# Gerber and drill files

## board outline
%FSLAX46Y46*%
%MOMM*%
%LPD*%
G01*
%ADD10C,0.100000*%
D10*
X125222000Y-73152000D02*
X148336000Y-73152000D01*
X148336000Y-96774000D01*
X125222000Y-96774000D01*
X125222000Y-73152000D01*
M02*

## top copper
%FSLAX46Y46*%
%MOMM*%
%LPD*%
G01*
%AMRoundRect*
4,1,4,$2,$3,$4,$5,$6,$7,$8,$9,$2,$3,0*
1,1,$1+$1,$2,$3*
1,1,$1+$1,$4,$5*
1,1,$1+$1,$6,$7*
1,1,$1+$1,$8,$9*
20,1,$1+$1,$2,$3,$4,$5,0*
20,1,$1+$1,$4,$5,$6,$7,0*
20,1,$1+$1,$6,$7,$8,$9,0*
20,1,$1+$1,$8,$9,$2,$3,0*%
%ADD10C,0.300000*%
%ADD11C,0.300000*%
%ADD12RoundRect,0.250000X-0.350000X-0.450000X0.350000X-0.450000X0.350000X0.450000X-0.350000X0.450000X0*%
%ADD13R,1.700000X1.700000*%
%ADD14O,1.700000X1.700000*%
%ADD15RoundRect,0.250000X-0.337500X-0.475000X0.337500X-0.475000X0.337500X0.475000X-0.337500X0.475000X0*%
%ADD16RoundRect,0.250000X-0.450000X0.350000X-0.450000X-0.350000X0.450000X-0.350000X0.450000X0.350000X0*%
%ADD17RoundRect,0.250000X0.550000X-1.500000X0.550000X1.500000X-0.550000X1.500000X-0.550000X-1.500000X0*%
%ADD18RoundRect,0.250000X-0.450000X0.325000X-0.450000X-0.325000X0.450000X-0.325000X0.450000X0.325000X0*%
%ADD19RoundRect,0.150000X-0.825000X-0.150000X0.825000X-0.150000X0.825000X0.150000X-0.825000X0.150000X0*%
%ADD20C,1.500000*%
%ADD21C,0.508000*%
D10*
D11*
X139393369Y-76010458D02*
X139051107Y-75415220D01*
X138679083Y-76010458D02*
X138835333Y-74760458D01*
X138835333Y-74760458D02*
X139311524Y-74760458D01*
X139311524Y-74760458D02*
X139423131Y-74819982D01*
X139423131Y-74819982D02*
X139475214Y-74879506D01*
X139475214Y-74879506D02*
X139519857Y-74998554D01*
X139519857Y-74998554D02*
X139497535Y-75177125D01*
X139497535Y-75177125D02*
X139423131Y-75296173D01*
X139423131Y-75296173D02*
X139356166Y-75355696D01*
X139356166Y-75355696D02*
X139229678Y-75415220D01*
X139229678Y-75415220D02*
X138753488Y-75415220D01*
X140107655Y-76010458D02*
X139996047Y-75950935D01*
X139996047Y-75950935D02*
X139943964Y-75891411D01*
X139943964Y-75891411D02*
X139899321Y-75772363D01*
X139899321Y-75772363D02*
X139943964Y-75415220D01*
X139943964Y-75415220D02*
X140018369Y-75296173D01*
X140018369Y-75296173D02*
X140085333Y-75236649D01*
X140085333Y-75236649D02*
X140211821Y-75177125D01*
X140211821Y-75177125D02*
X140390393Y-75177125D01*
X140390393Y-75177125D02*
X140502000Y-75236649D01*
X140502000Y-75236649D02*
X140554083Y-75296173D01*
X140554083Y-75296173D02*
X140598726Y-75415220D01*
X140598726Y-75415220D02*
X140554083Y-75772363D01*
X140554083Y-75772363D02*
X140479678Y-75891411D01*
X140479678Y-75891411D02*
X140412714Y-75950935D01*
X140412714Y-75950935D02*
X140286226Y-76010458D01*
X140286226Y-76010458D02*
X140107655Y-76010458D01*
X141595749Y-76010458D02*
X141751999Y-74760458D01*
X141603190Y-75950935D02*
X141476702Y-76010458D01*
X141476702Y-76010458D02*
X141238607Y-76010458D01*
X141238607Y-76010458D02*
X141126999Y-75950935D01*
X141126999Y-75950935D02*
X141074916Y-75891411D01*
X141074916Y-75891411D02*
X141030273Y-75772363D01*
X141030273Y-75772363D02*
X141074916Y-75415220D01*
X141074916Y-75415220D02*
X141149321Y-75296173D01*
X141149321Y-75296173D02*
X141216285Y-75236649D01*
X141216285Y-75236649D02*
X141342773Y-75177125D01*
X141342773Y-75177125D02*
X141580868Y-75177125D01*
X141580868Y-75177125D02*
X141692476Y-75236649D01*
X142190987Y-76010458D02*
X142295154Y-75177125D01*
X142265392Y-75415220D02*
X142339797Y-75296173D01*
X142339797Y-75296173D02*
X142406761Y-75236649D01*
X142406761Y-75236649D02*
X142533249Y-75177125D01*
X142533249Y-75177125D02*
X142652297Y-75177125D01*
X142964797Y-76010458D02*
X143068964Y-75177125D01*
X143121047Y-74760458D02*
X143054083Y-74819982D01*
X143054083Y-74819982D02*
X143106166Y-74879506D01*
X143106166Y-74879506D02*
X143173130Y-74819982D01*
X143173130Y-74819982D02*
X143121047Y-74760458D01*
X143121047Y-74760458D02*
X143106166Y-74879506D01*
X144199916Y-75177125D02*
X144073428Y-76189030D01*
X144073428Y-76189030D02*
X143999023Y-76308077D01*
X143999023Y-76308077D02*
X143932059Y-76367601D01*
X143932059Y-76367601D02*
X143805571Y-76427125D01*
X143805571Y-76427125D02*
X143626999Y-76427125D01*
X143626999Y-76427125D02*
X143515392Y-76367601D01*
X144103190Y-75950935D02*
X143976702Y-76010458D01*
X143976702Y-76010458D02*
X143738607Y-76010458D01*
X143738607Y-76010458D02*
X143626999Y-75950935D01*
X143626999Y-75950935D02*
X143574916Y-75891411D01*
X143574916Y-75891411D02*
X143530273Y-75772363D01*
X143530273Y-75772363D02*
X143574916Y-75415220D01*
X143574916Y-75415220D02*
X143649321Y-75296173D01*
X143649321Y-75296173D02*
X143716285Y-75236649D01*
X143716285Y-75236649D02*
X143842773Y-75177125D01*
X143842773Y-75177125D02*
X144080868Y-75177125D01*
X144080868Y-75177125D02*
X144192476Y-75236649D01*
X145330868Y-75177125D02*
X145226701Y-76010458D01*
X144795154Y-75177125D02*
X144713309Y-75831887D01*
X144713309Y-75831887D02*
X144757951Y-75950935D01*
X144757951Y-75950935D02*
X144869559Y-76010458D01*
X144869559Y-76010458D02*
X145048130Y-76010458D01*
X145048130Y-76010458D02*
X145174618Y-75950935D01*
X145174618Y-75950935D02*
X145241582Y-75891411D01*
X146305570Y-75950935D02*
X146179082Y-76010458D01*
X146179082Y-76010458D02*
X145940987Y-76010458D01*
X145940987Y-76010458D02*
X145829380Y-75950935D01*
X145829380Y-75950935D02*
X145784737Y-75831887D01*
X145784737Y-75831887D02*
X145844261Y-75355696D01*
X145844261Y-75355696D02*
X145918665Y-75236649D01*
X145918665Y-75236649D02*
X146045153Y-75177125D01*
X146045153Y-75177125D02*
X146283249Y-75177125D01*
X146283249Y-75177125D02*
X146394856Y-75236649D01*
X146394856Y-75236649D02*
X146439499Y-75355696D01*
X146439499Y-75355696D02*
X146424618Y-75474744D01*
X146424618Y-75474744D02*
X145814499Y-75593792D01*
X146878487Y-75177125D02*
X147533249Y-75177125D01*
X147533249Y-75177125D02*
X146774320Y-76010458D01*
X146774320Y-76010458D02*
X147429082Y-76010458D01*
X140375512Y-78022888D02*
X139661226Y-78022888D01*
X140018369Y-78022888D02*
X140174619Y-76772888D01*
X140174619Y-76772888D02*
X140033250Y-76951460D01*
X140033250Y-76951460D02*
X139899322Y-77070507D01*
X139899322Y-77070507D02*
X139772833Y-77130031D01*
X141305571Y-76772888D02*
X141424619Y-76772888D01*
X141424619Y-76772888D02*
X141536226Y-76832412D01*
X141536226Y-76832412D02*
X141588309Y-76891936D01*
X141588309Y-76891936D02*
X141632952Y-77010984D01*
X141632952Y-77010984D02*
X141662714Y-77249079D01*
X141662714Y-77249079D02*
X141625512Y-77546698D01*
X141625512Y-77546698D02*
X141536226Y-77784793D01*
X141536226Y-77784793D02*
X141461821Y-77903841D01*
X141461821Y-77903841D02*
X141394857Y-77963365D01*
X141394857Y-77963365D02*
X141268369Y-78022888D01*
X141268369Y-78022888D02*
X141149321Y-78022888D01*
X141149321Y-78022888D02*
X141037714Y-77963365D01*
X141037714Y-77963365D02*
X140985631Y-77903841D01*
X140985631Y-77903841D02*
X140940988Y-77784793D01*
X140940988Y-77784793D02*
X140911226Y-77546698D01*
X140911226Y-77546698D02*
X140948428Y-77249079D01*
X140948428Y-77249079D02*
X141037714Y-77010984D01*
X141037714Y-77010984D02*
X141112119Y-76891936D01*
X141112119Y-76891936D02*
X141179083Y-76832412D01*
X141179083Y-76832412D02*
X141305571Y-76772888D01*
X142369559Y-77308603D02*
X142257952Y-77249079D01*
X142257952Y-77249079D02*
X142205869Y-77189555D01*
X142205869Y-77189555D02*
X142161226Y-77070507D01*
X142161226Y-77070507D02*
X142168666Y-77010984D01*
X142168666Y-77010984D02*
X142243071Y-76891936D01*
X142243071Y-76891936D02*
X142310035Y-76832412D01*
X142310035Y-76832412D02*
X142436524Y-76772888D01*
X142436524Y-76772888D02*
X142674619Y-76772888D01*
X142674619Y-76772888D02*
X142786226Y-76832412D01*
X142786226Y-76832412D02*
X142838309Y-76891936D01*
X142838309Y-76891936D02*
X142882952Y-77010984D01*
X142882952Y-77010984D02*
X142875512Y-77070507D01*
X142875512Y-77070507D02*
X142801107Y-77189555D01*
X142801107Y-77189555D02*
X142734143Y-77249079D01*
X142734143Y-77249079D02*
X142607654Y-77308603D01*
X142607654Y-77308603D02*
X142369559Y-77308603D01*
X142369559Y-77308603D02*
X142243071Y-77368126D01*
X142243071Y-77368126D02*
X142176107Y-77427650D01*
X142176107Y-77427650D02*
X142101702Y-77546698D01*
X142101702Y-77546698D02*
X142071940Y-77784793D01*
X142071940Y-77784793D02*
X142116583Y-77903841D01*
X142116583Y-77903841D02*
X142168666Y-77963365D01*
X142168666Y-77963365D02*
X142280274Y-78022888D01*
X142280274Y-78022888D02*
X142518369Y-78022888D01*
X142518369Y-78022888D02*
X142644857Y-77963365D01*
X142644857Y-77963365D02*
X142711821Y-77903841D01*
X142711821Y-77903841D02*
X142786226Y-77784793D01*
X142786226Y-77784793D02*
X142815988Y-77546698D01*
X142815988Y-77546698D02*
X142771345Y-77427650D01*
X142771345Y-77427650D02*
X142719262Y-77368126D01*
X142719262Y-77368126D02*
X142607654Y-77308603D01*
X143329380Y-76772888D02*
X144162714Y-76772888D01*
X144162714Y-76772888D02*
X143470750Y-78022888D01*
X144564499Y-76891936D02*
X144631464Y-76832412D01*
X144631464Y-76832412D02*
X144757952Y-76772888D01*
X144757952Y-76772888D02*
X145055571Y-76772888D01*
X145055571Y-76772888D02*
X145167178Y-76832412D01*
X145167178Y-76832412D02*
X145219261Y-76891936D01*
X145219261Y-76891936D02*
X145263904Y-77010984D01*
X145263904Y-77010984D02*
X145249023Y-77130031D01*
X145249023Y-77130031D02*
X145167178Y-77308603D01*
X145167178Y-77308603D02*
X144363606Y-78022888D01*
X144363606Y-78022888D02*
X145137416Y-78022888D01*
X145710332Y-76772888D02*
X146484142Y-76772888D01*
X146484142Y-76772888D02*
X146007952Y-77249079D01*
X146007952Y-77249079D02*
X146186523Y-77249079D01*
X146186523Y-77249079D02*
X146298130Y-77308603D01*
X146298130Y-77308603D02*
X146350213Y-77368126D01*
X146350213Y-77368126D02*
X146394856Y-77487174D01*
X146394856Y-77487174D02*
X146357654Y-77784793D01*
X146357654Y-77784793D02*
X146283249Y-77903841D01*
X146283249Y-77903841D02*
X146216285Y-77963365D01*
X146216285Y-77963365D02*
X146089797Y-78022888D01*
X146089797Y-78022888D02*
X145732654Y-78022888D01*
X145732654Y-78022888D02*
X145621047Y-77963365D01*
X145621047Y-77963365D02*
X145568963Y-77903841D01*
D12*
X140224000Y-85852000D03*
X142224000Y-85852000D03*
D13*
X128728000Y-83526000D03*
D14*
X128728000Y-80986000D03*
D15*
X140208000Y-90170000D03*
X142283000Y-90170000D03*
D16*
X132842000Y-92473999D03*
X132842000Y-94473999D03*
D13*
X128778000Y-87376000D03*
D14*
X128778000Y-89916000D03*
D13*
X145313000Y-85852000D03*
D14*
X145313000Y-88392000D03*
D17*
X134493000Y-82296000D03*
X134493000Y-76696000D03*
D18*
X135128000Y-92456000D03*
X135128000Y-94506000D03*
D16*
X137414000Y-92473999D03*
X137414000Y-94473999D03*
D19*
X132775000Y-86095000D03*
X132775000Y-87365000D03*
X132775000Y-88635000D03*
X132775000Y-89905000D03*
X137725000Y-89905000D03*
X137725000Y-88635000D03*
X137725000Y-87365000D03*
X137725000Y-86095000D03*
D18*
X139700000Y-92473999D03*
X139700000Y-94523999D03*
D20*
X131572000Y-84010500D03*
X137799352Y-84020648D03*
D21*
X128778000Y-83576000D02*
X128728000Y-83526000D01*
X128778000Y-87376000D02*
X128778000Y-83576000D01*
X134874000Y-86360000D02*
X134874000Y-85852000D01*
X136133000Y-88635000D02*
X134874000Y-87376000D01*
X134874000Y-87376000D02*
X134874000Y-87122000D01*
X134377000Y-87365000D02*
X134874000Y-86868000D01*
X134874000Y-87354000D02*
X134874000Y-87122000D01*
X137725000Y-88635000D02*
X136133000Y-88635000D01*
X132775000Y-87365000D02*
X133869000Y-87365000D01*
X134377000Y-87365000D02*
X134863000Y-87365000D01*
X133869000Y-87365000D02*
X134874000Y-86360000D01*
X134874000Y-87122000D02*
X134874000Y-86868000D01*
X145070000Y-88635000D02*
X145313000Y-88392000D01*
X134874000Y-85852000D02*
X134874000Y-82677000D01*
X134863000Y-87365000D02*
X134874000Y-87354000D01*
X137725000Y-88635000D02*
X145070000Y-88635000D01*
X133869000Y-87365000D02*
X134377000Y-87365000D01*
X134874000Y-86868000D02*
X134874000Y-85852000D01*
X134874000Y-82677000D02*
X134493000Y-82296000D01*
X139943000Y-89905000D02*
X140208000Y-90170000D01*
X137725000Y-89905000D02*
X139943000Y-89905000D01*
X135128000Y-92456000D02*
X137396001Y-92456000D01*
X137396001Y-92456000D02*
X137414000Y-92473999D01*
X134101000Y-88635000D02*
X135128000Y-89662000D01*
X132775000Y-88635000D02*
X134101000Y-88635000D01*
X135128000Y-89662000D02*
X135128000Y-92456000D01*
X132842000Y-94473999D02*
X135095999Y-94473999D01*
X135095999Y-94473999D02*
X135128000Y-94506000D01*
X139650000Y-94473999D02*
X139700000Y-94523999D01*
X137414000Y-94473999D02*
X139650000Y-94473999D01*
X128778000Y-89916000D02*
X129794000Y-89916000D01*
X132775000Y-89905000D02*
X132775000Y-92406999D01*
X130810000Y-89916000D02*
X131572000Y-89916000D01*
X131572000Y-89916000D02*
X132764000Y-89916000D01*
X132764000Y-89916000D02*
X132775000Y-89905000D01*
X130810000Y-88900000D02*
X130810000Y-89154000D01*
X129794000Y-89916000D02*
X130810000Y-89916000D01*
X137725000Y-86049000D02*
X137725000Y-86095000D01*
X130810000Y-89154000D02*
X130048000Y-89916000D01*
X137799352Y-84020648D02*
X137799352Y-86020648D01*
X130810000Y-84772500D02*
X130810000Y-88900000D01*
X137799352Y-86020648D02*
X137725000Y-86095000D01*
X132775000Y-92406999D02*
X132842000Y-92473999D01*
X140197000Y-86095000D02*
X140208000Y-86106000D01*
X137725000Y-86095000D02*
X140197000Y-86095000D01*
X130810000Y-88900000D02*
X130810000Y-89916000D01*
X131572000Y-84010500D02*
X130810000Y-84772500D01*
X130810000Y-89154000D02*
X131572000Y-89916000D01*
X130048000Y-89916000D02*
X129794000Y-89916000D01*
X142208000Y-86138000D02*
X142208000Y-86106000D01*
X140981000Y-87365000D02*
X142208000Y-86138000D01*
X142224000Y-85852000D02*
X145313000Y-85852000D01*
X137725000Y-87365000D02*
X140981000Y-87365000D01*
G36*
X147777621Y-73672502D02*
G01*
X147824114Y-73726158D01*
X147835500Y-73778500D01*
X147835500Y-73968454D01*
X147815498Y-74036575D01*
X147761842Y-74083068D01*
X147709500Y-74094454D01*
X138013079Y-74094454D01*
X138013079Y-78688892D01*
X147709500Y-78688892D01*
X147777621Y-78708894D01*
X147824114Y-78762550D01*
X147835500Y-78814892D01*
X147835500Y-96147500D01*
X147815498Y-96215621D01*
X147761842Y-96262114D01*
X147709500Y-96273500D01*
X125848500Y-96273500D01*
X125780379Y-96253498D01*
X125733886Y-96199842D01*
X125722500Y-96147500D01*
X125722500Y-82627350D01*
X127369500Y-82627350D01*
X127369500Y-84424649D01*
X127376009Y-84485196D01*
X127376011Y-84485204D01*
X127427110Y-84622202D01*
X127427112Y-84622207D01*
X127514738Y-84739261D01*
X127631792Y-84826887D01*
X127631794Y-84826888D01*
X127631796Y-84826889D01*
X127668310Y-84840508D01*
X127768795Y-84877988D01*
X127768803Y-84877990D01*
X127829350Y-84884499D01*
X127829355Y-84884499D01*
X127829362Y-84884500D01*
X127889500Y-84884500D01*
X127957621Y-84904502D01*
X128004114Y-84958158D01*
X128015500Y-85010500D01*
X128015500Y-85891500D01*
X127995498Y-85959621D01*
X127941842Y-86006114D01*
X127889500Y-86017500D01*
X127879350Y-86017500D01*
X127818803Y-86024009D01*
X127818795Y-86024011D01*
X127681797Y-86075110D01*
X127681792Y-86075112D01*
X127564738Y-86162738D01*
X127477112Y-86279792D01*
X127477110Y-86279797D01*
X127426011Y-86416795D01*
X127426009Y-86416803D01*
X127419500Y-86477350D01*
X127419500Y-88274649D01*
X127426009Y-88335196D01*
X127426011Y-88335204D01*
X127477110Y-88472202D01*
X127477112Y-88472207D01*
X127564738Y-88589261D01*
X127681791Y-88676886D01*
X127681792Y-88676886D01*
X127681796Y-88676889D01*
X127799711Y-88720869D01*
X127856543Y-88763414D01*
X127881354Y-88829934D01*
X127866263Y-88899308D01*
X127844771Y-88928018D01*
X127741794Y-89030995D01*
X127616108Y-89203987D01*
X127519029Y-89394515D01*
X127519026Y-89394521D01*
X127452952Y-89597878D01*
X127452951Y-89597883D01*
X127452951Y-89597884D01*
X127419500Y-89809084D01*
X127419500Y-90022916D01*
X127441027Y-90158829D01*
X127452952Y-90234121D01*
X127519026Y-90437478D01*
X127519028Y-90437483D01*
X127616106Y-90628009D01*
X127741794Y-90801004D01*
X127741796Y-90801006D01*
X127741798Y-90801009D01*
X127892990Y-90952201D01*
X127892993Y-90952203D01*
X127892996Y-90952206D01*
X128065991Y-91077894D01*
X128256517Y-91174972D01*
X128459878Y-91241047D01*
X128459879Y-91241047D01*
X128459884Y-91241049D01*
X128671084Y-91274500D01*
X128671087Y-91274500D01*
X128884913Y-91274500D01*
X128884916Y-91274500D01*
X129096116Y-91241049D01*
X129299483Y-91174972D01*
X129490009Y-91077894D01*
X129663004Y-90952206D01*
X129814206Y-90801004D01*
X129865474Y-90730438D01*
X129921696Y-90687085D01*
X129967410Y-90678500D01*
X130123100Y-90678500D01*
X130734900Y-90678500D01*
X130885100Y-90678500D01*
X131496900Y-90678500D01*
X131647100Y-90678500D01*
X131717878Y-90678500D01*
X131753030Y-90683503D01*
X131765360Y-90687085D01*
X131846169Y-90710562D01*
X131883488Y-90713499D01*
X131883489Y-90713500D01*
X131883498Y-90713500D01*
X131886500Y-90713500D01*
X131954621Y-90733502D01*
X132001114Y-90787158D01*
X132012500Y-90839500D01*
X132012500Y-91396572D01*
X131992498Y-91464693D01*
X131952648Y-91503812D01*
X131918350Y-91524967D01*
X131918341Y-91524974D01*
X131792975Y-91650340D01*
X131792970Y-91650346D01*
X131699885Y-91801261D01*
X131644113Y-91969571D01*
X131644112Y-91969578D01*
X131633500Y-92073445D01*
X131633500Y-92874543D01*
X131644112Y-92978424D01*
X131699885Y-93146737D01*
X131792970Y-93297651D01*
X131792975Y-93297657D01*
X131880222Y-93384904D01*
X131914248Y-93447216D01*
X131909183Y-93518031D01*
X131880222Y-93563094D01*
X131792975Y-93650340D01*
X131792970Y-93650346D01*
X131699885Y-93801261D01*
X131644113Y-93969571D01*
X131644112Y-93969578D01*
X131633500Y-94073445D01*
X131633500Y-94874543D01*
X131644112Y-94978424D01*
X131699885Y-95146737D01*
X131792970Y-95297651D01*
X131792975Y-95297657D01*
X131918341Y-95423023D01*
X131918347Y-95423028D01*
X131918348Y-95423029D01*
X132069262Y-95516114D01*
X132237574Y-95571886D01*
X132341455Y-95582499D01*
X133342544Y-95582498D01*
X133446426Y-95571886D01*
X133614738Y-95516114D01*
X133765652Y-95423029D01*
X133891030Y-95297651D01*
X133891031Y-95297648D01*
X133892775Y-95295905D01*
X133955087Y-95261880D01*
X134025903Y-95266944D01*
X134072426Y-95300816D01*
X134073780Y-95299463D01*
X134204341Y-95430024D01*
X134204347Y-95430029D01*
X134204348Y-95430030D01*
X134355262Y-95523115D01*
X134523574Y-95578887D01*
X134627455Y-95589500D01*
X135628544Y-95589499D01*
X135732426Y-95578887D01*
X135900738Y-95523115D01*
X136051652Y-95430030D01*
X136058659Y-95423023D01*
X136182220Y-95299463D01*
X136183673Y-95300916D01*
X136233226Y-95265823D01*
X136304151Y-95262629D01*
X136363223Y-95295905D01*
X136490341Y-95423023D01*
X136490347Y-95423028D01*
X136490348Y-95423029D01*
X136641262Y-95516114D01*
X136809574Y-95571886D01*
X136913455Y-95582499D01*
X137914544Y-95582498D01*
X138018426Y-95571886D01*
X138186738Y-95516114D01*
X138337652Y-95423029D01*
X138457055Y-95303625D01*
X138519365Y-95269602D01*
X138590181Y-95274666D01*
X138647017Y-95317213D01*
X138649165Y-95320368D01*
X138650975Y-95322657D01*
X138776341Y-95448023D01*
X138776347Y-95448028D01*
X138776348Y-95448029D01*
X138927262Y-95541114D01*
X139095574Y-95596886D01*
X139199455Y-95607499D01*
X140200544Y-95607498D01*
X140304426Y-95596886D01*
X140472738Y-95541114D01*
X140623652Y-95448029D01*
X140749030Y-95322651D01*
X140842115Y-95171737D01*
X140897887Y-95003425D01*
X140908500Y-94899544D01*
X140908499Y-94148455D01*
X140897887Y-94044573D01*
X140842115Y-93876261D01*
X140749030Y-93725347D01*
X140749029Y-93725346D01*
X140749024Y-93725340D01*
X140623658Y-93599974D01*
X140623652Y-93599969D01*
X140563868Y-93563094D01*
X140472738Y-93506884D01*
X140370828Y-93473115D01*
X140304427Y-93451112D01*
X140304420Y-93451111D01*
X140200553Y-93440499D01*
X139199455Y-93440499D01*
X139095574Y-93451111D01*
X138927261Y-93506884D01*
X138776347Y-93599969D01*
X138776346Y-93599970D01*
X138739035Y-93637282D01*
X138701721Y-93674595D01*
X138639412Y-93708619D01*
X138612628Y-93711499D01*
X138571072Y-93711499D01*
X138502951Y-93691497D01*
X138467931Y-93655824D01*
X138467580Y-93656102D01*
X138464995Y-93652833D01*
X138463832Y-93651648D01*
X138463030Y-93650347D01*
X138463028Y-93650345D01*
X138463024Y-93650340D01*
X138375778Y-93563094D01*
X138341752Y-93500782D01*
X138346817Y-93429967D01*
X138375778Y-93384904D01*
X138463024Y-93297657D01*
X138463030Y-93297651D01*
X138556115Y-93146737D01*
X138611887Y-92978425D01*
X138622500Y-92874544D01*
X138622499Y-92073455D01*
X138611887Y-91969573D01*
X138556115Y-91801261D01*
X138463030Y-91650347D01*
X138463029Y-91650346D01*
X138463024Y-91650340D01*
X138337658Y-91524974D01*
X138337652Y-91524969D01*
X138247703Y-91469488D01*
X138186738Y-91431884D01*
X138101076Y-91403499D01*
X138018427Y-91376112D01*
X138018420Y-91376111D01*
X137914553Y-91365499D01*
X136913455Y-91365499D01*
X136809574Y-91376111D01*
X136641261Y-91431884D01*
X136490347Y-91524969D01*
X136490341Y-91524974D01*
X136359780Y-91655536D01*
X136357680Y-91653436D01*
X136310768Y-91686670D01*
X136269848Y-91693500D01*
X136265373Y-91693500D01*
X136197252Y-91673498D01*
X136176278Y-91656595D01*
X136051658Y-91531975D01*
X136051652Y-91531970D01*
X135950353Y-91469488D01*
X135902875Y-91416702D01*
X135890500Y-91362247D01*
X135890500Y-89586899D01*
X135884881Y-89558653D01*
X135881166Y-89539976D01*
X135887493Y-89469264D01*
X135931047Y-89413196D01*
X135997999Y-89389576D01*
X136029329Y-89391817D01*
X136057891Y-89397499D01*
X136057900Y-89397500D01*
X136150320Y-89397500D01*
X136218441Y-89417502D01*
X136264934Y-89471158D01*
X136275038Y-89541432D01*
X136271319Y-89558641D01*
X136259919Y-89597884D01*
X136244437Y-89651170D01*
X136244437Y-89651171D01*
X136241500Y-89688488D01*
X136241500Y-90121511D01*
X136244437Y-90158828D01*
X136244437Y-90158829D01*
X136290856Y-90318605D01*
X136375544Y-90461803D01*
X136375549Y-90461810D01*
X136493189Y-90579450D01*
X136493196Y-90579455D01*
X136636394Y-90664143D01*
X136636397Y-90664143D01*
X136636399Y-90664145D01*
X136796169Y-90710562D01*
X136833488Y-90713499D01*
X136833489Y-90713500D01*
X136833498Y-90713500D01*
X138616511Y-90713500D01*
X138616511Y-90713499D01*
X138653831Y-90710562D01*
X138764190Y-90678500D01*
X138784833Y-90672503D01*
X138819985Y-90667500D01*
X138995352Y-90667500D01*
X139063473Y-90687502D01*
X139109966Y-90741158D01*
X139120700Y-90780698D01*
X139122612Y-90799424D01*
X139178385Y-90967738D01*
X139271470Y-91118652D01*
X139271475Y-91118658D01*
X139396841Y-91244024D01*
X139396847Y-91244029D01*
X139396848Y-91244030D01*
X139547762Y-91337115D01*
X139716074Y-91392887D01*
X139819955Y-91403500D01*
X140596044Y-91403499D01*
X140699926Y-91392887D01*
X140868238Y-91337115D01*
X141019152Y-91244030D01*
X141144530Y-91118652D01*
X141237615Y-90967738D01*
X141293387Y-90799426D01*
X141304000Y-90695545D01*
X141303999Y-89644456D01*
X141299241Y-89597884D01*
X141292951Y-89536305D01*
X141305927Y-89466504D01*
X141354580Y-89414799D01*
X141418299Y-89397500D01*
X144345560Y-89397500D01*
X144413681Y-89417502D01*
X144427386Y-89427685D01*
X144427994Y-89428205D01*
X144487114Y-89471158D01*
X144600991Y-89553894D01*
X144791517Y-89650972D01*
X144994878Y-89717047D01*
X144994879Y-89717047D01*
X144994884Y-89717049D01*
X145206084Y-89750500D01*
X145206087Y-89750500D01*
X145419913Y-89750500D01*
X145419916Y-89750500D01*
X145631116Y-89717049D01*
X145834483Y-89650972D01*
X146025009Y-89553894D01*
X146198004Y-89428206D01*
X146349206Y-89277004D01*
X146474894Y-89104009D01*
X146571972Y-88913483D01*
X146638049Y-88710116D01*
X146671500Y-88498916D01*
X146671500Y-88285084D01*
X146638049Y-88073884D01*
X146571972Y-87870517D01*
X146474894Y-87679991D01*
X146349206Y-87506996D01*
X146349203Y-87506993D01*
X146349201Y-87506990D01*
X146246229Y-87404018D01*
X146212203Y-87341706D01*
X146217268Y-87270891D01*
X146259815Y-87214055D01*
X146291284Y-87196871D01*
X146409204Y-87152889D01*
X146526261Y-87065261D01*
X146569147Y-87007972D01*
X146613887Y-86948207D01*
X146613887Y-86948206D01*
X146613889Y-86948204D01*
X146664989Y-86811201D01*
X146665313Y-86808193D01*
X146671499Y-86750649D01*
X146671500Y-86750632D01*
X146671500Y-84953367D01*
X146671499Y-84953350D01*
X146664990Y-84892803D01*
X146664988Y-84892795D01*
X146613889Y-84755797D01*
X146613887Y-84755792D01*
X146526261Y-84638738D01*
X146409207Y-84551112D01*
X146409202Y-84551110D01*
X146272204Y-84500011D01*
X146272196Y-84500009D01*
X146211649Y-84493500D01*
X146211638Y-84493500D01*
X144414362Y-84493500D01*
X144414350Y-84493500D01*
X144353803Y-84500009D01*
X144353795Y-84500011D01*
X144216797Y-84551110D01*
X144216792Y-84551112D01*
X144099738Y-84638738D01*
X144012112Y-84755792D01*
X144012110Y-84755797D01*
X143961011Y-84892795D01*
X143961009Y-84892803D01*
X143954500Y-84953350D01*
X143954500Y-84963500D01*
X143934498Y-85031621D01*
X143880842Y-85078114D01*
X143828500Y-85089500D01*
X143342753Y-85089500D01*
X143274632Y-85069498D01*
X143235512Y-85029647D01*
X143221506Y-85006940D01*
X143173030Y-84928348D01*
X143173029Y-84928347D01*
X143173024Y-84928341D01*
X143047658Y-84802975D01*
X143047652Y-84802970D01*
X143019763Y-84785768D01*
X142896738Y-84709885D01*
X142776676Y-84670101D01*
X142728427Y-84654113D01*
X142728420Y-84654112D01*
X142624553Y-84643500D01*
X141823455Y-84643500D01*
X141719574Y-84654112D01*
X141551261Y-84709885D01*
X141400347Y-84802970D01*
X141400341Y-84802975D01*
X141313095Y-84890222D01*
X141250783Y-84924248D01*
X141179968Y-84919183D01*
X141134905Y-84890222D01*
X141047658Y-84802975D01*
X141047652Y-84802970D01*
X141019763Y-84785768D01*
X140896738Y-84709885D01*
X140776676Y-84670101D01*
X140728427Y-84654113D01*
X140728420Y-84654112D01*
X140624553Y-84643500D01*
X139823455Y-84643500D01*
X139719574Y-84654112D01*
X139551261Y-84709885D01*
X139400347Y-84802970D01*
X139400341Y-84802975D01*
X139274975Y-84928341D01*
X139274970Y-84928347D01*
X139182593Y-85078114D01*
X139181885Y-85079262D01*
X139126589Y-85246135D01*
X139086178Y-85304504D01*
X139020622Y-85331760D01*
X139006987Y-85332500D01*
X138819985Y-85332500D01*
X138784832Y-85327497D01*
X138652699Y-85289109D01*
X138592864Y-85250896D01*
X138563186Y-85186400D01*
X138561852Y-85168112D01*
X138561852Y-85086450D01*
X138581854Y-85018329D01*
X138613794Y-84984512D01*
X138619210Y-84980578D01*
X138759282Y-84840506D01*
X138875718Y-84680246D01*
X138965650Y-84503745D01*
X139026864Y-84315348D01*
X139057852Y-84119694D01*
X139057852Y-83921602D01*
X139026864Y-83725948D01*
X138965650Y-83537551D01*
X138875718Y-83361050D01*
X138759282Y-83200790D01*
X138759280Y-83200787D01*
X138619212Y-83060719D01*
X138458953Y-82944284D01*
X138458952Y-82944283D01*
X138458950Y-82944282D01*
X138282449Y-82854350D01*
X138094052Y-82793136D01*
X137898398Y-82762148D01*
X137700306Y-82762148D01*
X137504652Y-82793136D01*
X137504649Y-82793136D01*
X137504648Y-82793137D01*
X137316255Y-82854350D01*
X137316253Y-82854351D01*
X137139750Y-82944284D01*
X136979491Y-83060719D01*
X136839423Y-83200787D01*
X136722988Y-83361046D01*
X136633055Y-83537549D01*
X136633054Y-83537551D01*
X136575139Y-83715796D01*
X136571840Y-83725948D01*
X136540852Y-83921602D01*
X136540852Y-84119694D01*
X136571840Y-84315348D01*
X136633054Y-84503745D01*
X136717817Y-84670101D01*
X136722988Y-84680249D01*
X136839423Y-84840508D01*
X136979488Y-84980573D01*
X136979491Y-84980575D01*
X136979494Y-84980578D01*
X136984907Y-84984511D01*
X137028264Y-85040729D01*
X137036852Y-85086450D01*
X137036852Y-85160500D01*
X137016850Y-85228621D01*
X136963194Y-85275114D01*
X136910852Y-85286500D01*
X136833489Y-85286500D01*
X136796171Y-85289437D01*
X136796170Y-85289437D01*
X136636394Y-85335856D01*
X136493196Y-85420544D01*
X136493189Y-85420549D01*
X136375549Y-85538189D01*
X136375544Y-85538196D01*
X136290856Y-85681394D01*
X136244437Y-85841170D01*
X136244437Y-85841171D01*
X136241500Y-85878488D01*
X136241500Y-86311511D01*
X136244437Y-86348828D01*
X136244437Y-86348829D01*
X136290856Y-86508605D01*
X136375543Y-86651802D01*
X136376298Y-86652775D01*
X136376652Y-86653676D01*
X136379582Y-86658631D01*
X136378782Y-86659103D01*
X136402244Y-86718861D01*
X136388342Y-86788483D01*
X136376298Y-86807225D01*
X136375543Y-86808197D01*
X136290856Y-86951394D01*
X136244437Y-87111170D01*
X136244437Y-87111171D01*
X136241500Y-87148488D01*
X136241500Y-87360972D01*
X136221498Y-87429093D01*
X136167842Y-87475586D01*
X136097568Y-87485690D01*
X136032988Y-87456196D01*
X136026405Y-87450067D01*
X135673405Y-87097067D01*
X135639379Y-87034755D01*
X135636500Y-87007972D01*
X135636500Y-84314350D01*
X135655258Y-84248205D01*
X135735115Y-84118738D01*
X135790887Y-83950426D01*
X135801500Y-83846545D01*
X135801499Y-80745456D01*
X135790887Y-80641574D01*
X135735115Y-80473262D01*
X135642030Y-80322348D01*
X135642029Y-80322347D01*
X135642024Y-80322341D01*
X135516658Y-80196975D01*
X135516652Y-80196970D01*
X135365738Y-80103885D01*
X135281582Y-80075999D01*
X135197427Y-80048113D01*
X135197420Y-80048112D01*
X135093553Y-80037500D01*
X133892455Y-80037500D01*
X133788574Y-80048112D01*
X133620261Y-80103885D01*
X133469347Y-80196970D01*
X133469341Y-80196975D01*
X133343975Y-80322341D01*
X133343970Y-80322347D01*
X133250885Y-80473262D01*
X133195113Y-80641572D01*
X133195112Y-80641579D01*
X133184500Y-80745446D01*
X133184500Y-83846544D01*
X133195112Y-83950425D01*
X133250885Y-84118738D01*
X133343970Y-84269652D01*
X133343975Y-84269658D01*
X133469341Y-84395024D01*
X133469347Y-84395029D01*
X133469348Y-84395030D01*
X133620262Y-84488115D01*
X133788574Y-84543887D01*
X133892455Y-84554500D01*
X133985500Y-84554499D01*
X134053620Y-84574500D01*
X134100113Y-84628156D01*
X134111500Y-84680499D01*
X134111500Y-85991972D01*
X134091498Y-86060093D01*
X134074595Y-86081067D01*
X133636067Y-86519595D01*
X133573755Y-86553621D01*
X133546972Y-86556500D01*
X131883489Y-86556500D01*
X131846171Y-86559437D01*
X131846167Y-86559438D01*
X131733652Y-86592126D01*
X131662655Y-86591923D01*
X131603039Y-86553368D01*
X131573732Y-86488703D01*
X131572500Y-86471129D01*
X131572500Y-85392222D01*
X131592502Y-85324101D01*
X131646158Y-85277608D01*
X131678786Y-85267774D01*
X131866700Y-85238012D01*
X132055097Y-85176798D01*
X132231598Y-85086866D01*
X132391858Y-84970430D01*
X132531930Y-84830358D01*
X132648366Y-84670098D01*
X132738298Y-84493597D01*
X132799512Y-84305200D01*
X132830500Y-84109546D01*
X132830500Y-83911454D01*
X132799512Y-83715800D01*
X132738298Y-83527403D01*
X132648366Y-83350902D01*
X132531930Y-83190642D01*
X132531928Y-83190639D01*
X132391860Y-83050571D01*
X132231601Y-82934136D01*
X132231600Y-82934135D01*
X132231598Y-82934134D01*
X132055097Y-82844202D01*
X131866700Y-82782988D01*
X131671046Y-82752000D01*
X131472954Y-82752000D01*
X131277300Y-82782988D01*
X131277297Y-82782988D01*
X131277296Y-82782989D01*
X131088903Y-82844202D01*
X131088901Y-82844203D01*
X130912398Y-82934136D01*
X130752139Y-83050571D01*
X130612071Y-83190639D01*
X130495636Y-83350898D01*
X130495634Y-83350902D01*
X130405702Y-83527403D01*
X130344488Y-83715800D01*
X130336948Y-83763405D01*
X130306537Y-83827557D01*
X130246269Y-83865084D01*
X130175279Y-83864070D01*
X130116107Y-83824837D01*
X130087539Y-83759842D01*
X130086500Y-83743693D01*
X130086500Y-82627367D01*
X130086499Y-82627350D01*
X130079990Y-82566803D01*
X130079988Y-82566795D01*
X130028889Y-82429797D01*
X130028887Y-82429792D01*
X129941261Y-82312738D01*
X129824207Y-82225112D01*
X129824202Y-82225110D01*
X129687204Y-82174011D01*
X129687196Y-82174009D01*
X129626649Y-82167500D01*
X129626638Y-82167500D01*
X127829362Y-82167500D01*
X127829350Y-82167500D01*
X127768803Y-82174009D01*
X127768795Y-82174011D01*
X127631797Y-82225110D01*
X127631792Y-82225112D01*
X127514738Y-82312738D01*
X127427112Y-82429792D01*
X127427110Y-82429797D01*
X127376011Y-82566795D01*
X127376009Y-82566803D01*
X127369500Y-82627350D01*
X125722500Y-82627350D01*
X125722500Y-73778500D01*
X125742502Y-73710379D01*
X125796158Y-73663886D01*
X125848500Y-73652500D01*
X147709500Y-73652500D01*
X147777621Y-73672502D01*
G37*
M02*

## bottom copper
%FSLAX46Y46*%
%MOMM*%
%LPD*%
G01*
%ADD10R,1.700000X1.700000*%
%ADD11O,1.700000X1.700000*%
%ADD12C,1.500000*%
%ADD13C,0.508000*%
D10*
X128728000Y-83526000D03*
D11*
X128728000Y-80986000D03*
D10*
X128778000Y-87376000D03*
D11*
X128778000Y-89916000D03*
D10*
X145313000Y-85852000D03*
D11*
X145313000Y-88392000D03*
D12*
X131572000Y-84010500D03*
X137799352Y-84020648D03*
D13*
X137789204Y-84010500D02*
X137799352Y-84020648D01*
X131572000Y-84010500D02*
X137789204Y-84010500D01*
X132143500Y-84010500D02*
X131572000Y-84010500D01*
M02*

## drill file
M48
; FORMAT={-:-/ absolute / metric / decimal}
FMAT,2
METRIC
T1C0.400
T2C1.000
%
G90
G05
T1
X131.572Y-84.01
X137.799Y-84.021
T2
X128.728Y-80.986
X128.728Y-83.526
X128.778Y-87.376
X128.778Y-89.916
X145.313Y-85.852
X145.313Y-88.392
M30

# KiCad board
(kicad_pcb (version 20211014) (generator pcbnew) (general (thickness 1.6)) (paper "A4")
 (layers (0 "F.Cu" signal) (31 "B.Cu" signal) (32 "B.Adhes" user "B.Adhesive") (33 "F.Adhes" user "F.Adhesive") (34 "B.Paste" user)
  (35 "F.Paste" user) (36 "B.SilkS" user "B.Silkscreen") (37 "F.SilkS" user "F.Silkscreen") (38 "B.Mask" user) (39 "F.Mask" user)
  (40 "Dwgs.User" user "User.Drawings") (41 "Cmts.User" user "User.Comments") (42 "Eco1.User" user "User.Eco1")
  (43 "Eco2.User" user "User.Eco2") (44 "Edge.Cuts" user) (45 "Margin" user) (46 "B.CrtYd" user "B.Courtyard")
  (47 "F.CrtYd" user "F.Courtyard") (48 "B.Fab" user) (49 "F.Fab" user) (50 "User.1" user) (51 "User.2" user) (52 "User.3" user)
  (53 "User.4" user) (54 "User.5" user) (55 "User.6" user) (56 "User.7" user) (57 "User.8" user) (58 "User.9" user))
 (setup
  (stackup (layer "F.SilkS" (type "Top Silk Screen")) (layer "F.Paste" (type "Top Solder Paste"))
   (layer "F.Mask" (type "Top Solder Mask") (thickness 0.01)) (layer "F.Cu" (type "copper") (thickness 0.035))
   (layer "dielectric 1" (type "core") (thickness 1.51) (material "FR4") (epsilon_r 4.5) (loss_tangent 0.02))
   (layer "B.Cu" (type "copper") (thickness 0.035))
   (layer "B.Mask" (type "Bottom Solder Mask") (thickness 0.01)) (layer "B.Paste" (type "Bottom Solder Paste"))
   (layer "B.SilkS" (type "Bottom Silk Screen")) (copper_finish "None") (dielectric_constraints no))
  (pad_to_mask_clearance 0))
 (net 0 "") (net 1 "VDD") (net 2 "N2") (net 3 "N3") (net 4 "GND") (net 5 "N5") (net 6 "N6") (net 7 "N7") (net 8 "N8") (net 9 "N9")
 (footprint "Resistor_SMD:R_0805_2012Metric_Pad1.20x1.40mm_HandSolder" (layer "F.Cu") (at 141.224 85.852)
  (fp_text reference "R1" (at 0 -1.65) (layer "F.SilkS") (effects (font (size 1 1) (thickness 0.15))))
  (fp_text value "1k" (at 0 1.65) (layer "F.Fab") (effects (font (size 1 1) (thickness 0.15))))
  (pad "1" smd roundrect (at -1 0) (size 1.2 1.4) (layers "F.Cu" "F.Paste" "F.Mask") (roundrect_rratio 0.208333) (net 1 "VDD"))
  (pad "2" smd roundrect (at 1 0) (size 1.2 1.4) (layers "F.Cu" "F.Paste" "F.Mask") (roundrect_rratio 0.208333) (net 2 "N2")))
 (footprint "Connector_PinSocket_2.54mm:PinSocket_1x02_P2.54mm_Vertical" (layer "F.Cu") (at 128.728 83.526 180)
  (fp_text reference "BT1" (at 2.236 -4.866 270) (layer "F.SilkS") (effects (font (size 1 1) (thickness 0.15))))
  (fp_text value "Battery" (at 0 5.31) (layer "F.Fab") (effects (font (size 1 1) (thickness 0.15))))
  (pad "1" thru_hole rect (at 0 0 180) (size 1.7 1.7) (drill 1) (layers *.Cu *.Mask) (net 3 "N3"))
  (pad "2" thru_hole oval (at 0 2.54 180) (size 1.7 1.7) (drill 1) (layers *.Cu *.Mask) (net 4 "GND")))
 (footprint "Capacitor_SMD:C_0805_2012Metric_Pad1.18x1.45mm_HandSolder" (layer "F.Cu") (at 141.2455 90.17)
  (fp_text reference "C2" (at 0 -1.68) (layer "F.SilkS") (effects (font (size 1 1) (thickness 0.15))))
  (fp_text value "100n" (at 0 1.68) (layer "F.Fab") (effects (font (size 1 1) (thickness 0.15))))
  (pad "1" smd roundrect (at -1.0375 0) (size 1.175 1.45) (layers "F.Cu" "F.Paste" "F.Mask") (roundrect_rratio 0.212766) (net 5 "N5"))
  (pad "2" smd roundrect (at 1.0375 0) (size 1.175 1.45) (layers "F.Cu" "F.Paste" "F.Mask") (roundrect_rratio 0.212766) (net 4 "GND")))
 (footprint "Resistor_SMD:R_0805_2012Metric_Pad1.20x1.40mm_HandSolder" (layer "F.Cu") (at 132.842 93.473999 -90)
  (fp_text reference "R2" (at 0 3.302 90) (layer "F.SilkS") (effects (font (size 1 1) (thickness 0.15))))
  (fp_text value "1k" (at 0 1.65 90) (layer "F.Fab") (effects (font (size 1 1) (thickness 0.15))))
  (pad "1" smd roundrect (at -1 0 270) (size 1.2 1.4) (layers "F.Cu" "F.Paste" "F.Mask") (roundrect_rratio 0.208333) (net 1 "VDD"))
  (pad "2" smd roundrect (at 1 0 270) (size 1.2 1.4) (layers "F.Cu" "F.Paste" "F.Mask") (roundrect_rratio 0.208333) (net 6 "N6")))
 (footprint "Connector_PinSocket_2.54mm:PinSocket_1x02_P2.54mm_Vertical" (layer "F.Cu") (at 128.778 87.376)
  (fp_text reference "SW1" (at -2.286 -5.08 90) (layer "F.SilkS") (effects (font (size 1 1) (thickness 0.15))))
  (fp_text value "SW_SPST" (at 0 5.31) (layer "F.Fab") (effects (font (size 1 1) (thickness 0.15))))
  (pad "1" thru_hole rect (at 0 0) (size 1.7 1.7) (drill 1) (layers *.Cu *.Mask) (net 3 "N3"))
  (pad "2" thru_hole oval (at 0 2.54) (size 1.7 1.7) (drill 1) (layers *.Cu *.Mask) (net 1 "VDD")))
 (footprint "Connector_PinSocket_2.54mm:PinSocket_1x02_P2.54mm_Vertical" (layer "F.Cu") (at 145.313 85.852)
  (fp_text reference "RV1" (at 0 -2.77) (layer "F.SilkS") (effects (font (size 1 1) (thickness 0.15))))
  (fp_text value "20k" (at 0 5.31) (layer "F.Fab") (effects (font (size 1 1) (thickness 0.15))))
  (pad "1" thru_hole rect (at 0 0) (size 1.7 1.7) (drill 1) (layers *.Cu *.Mask) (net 2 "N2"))
  (pad "2" thru_hole oval (at 0 2.54) (size 1.7 1.7) (drill 1) (layers *.Cu *.Mask) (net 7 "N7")))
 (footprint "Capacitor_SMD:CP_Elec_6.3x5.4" (layer "F.Cu") (at 134.493 79.496 90)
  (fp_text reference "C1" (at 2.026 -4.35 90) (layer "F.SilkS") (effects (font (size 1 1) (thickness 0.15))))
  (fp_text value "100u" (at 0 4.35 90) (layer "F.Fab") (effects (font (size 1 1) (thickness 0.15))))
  (pad "1" smd roundrect (at -2.8 0 90) (size 3.5 1.6) (layers "F.Cu" "F.Paste" "F.Mask") (roundrect_rratio 0.15625) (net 7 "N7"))
  (pad "2" smd roundrect (at 2.8 0 90) (size 3.5 1.6) (layers "F.Cu" "F.Paste" "F.Mask") (roundrect_rratio 0.15625) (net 4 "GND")))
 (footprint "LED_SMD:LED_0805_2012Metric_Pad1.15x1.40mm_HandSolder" (layer "F.Cu") (at 135.128 93.481 -90)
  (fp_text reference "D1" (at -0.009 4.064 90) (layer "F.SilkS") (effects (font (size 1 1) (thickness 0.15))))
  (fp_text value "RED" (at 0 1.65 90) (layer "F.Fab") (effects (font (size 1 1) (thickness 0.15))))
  (pad "1" smd roundrect (at -1.025 0 270) (size 1.15 1.4) (layers "F.Cu" "F.Paste" "F.Mask") (roundrect_rratio 0.217391) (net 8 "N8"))
  (pad "2" smd roundrect (at 1.025 0 270) (size 1.15 1.4) (layers "F.Cu" "F.Paste" "F.Mask") (roundrect_rratio 0.217391) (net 6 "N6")))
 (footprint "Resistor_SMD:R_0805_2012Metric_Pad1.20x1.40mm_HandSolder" (layer "F.Cu") (at 137.414 93.473999 -90)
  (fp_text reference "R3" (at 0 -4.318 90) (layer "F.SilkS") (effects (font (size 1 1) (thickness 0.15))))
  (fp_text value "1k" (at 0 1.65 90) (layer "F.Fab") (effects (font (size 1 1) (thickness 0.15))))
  (pad "1" smd roundrect (at -1 0 270) (size 1.2 1.4) (layers "F.Cu" "F.Paste" "F.Mask") (roundrect_rratio 0.208333) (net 8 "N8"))
  (pad "2" smd roundrect (at 1 0 270) (size 1.2 1.4) (layers "F.Cu" "F.Paste" "F.Mask") (roundrect_rratio 0.208333) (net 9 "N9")))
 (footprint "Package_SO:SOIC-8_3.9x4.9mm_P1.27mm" (layer "F.Cu") (at 135.25 88)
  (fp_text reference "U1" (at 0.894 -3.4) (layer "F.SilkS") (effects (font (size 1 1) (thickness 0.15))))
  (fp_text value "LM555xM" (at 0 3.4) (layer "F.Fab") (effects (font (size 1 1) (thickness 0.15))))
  (pad "1" smd roundrect (at -2.475 -1.905) (size 1.95 0.6) (layers "F.Cu" "F.Paste" "F.Mask") (roundrect_rratio 0.25) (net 4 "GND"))
  (pad "2" smd roundrect (at -2.475 -0.635) (size 1.95 0.6) (layers "F.Cu" "F.Paste" "F.Mask") (roundrect_rratio 0.25) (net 7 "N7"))
  (pad "3" smd roundrect (at -2.475 0.635) (size 1.95 0.6) (layers "F.Cu" "F.Paste" "F.Mask") (roundrect_rratio 0.25) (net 8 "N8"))
  (pad "4" smd roundrect (at -2.475 1.905) (size 1.95 0.6) (layers "F.Cu" "F.Paste" "F.Mask") (roundrect_rratio 0.25) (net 1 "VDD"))
  (pad "5" smd roundrect (at 2.475 1.905) (size 1.95 0.6) (layers "F.Cu" "F.Paste" "F.Mask") (roundrect_rratio 0.25) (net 5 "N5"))
  (pad "6" smd roundrect (at 2.475 0.635) (size 1.95 0.6) (layers "F.Cu" "F.Paste" "F.Mask") (roundrect_rratio 0.25) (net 7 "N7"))
  (pad "7" smd roundrect (at 2.475 -0.635) (size 1.95 0.6) (layers "F.Cu" "F.Paste" "F.Mask") (roundrect_rratio 0.25) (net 2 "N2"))
  (pad "8" smd roundrect (at 2.475 -1.905) (size 1.95 0.6) (layers "F.Cu" "F.Paste" "F.Mask") (roundrect_rratio 0.25) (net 1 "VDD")))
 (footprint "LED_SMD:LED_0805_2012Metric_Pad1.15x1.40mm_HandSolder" (layer "F.Cu") (at 139.7 93.498999 -90)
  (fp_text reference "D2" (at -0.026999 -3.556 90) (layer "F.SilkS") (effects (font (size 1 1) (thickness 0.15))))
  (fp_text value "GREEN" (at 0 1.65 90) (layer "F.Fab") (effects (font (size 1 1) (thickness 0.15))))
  (pad "1" smd roundrect (at -1.025 0 270) (size 1.15 1.4) (layers "F.Cu" "F.Paste" "F.Mask") (roundrect_rratio 0.217391) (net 4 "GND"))
  (pad "2" smd roundrect (at 1.025 0 270) (size 1.15 1.4) (layers "F.Cu" "F.Paste" "F.Mask") (roundrect_rratio 0.217391) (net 9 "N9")))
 (gr_rect (start 125.222 73.152) (end 148.336 96.774) (layer "Edge.Cuts") (width 0.1) (fill none))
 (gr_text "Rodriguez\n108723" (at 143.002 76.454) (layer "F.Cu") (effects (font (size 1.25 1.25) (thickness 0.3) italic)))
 (segment (start 128.778 83.576) (end 128.728 83.526) (width 0.508) (layer "F.Cu") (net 3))
 (segment (start 128.778 87.376) (end 128.778 83.576) (width 0.508) (layer "F.Cu") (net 3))
 (segment (start 134.874 86.36) (end 134.874 85.852) (width 0.508) (layer "F.Cu") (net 7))
 (segment (start 136.133 88.635) (end 134.874 87.376) (width 0.508) (layer "F.Cu") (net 7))
 (segment (start 134.874 87.376) (end 134.874 87.122) (width 0.508) (layer "F.Cu") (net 7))
 (segment (start 134.377 87.365) (end 134.874 86.868) (width 0.508) (layer "F.Cu") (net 7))
 (segment (start 134.874 87.354) (end 134.874 87.122) (width 0.508) (layer "F.Cu") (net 7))
 (segment (start 137.725 88.635) (end 136.133 88.635) (width 0.508) (layer "F.Cu") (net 7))
 (segment (start 132.775 87.365) (end 133.869 87.365) (width 0.508) (layer "F.Cu") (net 7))
 (segment (start 134.377 87.365) (end 134.863 87.365) (width 0.508) (layer "F.Cu") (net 7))
 (segment (start 133.869 87.365) (end 134.874 86.36) (width 0.508) (layer "F.Cu") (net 7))
 (segment (start 134.874 87.122) (end 134.874 86.868) (width 0.508) (layer "F.Cu") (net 7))
 (segment (start 145.07 88.635) (end 145.313 88.392) (width 0.508) (layer "F.Cu") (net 7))
 (segment (start 134.874 85.852) (end 134.874 82.677) (width 0.508) (layer "F.Cu") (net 7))
 (segment (start 134.863 87.365) (end 134.874 87.354) (width 0.508) (layer "F.Cu") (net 7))
 (segment (start 137.725 88.635) (end 145.07 88.635) (width 0.508) (layer "F.Cu") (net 7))
 (segment (start 133.869 87.365) (end 134.377 87.365) (width 0.508) (layer "F.Cu") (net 7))
 (segment (start 134.874 86.868) (end 134.874 85.852) (width 0.508) (layer "F.Cu") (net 7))
 (segment (start 134.874 82.677) (end 134.493 82.296) (width 0.508) (layer "F.Cu") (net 7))
 (segment (start 139.943 89.905) (end 140.208 90.17) (width 0.508) (layer "F.Cu") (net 5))
 (segment (start 137.725 89.905) (end 139.943 89.905) (width 0.508) (layer "F.Cu") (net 5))
 (segment (start 135.128 92.456) (end 137.396001 92.456) (width 0.508) (layer "F.Cu") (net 8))
 (segment (start 137.396001 92.456) (end 137.414 92.473999) (width 0.508) (layer "F.Cu") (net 8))
 (segment (start 134.101 88.635) (end 135.128 89.662) (width 0.508) (layer "F.Cu") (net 8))
 (segment (start 132.775 88.635) (end 134.101 88.635) (width 0.508) (layer "F.Cu") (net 8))
 (segment (start 135.128 89.662) (end 135.128 92.456) (width 0.508) (layer "F.Cu") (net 8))
 (segment (start 132.842 94.473999) (end 135.095999 94.473999) (width 0.508) (layer "F.Cu") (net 6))
 (segment (start 135.095999 94.473999) (end 135.128 94.506) (width 0.508) (layer "F.Cu") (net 6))
 (segment (start 139.65 94.473999) (end 139.7 94.523999) (width 0.508) (layer "F.Cu") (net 9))
 (segment (start 137.414 94.473999) (end 139.65 94.473999) (width 0.508) (layer "F.Cu") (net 9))
 (segment (start 128.778 89.916) (end 129.794 89.916) (width 0.508) (layer "F.Cu") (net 1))
 (segment (start 132.775 89.905) (end 132.775 92.406999) (width 0.508) (layer "F.Cu") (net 1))
 (segment (start 130.81 89.916) (end 131.572 89.916) (width 0.508) (layer "F.Cu") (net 1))
 (segment (start 131.572 89.916) (end 132.764 89.916) (width 0.508) (layer "F.Cu") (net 1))
 (segment (start 132.764 89.916) (end 132.775 89.905) (width 0.508) (layer "F.Cu") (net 1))
 (segment (start 130.81 88.9) (end 130.81 89.154) (width 0.508) (layer "F.Cu") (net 1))
 (segment (start 129.794 89.916) (end 130.81 89.916) (width 0.508) (layer "F.Cu") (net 1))
 (segment (start 137.725 86.049) (end 137.725 86.095) (width 0.508) (layer "F.Cu") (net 1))
 (segment (start 130.81 89.154) (end 130.048 89.916) (width 0.508) (layer "F.Cu") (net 1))
 (segment (start 137.799352 84.020648) (end 137.799352 86.020648) (width 0.508) (layer "F.Cu") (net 1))
 (segment (start 130.81 84.7725) (end 130.81 88.9) (width 0.508) (layer "F.Cu") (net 1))
 (segment (start 137.799352 86.020648) (end 137.725 86.095) (width 0.508) (layer "F.Cu") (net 1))
 (segment (start 132.775 92.406999) (end 132.842 92.473999) (width 0.508) (layer "F.Cu") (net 1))
 (segment (start 140.197 86.095) (end 140.208 86.106) (width 0.508) (layer "F.Cu") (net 1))
 (segment (start 137.725 86.095) (end 140.197 86.095) (width 0.508) (layer "F.Cu") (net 1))
 (segment (start 130.81 88.9) (end 130.81 89.916) (width 0.508) (layer "F.Cu") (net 1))
 (segment (start 131.572 84.0105) (end 130.81 84.7725) (width 0.508) (layer "F.Cu") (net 1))
 (segment (start 130.81 89.154) (end 131.572 89.916) (width 0.508) (layer "F.Cu") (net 1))
 (segment (start 130.048 89.916) (end 129.794 89.916) (width 0.508) (layer "F.Cu") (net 1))
 (via (at 131.572 84.0105) (size 1.5) (drill 0.4) (layers "F.Cu" "B.Cu") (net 1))
 (via (at 137.799352 84.020648) (size 1.5) (drill 0.4) (layers "F.Cu" "B.Cu") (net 1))
 (segment (start 137.789204 84.0105) (end 137.799352 84.020648) (width 0.508) (layer "B.Cu") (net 1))
 (segment (start 131.572 84.0105) (end 137.789204 84.0105) (width 0.508) (layer "B.Cu") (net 1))
 (segment (start 132.1435 84.0105) (end 131.572 84.0105) (width 0.508) (layer "B.Cu") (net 1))
 (segment (start 142.208 86.138) (end 142.208 86.106) (width 0.508) (layer "F.Cu") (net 2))
 (segment (start 140.981 87.365) (end 142.208 86.138) (width 0.508) (layer "F.Cu") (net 2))
 (segment (start 142.224 85.852) (end 145.313 85.852) (width 0.508) (layer "F.Cu") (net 2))
 (segment (start 137.725 87.365) (end 140.981 87.365) (width 0.508) (layer "F.Cu") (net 2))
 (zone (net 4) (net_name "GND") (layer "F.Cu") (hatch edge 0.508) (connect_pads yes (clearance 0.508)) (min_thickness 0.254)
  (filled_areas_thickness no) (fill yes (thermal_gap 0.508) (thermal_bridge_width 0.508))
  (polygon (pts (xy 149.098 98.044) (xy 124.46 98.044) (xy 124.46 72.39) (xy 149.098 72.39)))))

